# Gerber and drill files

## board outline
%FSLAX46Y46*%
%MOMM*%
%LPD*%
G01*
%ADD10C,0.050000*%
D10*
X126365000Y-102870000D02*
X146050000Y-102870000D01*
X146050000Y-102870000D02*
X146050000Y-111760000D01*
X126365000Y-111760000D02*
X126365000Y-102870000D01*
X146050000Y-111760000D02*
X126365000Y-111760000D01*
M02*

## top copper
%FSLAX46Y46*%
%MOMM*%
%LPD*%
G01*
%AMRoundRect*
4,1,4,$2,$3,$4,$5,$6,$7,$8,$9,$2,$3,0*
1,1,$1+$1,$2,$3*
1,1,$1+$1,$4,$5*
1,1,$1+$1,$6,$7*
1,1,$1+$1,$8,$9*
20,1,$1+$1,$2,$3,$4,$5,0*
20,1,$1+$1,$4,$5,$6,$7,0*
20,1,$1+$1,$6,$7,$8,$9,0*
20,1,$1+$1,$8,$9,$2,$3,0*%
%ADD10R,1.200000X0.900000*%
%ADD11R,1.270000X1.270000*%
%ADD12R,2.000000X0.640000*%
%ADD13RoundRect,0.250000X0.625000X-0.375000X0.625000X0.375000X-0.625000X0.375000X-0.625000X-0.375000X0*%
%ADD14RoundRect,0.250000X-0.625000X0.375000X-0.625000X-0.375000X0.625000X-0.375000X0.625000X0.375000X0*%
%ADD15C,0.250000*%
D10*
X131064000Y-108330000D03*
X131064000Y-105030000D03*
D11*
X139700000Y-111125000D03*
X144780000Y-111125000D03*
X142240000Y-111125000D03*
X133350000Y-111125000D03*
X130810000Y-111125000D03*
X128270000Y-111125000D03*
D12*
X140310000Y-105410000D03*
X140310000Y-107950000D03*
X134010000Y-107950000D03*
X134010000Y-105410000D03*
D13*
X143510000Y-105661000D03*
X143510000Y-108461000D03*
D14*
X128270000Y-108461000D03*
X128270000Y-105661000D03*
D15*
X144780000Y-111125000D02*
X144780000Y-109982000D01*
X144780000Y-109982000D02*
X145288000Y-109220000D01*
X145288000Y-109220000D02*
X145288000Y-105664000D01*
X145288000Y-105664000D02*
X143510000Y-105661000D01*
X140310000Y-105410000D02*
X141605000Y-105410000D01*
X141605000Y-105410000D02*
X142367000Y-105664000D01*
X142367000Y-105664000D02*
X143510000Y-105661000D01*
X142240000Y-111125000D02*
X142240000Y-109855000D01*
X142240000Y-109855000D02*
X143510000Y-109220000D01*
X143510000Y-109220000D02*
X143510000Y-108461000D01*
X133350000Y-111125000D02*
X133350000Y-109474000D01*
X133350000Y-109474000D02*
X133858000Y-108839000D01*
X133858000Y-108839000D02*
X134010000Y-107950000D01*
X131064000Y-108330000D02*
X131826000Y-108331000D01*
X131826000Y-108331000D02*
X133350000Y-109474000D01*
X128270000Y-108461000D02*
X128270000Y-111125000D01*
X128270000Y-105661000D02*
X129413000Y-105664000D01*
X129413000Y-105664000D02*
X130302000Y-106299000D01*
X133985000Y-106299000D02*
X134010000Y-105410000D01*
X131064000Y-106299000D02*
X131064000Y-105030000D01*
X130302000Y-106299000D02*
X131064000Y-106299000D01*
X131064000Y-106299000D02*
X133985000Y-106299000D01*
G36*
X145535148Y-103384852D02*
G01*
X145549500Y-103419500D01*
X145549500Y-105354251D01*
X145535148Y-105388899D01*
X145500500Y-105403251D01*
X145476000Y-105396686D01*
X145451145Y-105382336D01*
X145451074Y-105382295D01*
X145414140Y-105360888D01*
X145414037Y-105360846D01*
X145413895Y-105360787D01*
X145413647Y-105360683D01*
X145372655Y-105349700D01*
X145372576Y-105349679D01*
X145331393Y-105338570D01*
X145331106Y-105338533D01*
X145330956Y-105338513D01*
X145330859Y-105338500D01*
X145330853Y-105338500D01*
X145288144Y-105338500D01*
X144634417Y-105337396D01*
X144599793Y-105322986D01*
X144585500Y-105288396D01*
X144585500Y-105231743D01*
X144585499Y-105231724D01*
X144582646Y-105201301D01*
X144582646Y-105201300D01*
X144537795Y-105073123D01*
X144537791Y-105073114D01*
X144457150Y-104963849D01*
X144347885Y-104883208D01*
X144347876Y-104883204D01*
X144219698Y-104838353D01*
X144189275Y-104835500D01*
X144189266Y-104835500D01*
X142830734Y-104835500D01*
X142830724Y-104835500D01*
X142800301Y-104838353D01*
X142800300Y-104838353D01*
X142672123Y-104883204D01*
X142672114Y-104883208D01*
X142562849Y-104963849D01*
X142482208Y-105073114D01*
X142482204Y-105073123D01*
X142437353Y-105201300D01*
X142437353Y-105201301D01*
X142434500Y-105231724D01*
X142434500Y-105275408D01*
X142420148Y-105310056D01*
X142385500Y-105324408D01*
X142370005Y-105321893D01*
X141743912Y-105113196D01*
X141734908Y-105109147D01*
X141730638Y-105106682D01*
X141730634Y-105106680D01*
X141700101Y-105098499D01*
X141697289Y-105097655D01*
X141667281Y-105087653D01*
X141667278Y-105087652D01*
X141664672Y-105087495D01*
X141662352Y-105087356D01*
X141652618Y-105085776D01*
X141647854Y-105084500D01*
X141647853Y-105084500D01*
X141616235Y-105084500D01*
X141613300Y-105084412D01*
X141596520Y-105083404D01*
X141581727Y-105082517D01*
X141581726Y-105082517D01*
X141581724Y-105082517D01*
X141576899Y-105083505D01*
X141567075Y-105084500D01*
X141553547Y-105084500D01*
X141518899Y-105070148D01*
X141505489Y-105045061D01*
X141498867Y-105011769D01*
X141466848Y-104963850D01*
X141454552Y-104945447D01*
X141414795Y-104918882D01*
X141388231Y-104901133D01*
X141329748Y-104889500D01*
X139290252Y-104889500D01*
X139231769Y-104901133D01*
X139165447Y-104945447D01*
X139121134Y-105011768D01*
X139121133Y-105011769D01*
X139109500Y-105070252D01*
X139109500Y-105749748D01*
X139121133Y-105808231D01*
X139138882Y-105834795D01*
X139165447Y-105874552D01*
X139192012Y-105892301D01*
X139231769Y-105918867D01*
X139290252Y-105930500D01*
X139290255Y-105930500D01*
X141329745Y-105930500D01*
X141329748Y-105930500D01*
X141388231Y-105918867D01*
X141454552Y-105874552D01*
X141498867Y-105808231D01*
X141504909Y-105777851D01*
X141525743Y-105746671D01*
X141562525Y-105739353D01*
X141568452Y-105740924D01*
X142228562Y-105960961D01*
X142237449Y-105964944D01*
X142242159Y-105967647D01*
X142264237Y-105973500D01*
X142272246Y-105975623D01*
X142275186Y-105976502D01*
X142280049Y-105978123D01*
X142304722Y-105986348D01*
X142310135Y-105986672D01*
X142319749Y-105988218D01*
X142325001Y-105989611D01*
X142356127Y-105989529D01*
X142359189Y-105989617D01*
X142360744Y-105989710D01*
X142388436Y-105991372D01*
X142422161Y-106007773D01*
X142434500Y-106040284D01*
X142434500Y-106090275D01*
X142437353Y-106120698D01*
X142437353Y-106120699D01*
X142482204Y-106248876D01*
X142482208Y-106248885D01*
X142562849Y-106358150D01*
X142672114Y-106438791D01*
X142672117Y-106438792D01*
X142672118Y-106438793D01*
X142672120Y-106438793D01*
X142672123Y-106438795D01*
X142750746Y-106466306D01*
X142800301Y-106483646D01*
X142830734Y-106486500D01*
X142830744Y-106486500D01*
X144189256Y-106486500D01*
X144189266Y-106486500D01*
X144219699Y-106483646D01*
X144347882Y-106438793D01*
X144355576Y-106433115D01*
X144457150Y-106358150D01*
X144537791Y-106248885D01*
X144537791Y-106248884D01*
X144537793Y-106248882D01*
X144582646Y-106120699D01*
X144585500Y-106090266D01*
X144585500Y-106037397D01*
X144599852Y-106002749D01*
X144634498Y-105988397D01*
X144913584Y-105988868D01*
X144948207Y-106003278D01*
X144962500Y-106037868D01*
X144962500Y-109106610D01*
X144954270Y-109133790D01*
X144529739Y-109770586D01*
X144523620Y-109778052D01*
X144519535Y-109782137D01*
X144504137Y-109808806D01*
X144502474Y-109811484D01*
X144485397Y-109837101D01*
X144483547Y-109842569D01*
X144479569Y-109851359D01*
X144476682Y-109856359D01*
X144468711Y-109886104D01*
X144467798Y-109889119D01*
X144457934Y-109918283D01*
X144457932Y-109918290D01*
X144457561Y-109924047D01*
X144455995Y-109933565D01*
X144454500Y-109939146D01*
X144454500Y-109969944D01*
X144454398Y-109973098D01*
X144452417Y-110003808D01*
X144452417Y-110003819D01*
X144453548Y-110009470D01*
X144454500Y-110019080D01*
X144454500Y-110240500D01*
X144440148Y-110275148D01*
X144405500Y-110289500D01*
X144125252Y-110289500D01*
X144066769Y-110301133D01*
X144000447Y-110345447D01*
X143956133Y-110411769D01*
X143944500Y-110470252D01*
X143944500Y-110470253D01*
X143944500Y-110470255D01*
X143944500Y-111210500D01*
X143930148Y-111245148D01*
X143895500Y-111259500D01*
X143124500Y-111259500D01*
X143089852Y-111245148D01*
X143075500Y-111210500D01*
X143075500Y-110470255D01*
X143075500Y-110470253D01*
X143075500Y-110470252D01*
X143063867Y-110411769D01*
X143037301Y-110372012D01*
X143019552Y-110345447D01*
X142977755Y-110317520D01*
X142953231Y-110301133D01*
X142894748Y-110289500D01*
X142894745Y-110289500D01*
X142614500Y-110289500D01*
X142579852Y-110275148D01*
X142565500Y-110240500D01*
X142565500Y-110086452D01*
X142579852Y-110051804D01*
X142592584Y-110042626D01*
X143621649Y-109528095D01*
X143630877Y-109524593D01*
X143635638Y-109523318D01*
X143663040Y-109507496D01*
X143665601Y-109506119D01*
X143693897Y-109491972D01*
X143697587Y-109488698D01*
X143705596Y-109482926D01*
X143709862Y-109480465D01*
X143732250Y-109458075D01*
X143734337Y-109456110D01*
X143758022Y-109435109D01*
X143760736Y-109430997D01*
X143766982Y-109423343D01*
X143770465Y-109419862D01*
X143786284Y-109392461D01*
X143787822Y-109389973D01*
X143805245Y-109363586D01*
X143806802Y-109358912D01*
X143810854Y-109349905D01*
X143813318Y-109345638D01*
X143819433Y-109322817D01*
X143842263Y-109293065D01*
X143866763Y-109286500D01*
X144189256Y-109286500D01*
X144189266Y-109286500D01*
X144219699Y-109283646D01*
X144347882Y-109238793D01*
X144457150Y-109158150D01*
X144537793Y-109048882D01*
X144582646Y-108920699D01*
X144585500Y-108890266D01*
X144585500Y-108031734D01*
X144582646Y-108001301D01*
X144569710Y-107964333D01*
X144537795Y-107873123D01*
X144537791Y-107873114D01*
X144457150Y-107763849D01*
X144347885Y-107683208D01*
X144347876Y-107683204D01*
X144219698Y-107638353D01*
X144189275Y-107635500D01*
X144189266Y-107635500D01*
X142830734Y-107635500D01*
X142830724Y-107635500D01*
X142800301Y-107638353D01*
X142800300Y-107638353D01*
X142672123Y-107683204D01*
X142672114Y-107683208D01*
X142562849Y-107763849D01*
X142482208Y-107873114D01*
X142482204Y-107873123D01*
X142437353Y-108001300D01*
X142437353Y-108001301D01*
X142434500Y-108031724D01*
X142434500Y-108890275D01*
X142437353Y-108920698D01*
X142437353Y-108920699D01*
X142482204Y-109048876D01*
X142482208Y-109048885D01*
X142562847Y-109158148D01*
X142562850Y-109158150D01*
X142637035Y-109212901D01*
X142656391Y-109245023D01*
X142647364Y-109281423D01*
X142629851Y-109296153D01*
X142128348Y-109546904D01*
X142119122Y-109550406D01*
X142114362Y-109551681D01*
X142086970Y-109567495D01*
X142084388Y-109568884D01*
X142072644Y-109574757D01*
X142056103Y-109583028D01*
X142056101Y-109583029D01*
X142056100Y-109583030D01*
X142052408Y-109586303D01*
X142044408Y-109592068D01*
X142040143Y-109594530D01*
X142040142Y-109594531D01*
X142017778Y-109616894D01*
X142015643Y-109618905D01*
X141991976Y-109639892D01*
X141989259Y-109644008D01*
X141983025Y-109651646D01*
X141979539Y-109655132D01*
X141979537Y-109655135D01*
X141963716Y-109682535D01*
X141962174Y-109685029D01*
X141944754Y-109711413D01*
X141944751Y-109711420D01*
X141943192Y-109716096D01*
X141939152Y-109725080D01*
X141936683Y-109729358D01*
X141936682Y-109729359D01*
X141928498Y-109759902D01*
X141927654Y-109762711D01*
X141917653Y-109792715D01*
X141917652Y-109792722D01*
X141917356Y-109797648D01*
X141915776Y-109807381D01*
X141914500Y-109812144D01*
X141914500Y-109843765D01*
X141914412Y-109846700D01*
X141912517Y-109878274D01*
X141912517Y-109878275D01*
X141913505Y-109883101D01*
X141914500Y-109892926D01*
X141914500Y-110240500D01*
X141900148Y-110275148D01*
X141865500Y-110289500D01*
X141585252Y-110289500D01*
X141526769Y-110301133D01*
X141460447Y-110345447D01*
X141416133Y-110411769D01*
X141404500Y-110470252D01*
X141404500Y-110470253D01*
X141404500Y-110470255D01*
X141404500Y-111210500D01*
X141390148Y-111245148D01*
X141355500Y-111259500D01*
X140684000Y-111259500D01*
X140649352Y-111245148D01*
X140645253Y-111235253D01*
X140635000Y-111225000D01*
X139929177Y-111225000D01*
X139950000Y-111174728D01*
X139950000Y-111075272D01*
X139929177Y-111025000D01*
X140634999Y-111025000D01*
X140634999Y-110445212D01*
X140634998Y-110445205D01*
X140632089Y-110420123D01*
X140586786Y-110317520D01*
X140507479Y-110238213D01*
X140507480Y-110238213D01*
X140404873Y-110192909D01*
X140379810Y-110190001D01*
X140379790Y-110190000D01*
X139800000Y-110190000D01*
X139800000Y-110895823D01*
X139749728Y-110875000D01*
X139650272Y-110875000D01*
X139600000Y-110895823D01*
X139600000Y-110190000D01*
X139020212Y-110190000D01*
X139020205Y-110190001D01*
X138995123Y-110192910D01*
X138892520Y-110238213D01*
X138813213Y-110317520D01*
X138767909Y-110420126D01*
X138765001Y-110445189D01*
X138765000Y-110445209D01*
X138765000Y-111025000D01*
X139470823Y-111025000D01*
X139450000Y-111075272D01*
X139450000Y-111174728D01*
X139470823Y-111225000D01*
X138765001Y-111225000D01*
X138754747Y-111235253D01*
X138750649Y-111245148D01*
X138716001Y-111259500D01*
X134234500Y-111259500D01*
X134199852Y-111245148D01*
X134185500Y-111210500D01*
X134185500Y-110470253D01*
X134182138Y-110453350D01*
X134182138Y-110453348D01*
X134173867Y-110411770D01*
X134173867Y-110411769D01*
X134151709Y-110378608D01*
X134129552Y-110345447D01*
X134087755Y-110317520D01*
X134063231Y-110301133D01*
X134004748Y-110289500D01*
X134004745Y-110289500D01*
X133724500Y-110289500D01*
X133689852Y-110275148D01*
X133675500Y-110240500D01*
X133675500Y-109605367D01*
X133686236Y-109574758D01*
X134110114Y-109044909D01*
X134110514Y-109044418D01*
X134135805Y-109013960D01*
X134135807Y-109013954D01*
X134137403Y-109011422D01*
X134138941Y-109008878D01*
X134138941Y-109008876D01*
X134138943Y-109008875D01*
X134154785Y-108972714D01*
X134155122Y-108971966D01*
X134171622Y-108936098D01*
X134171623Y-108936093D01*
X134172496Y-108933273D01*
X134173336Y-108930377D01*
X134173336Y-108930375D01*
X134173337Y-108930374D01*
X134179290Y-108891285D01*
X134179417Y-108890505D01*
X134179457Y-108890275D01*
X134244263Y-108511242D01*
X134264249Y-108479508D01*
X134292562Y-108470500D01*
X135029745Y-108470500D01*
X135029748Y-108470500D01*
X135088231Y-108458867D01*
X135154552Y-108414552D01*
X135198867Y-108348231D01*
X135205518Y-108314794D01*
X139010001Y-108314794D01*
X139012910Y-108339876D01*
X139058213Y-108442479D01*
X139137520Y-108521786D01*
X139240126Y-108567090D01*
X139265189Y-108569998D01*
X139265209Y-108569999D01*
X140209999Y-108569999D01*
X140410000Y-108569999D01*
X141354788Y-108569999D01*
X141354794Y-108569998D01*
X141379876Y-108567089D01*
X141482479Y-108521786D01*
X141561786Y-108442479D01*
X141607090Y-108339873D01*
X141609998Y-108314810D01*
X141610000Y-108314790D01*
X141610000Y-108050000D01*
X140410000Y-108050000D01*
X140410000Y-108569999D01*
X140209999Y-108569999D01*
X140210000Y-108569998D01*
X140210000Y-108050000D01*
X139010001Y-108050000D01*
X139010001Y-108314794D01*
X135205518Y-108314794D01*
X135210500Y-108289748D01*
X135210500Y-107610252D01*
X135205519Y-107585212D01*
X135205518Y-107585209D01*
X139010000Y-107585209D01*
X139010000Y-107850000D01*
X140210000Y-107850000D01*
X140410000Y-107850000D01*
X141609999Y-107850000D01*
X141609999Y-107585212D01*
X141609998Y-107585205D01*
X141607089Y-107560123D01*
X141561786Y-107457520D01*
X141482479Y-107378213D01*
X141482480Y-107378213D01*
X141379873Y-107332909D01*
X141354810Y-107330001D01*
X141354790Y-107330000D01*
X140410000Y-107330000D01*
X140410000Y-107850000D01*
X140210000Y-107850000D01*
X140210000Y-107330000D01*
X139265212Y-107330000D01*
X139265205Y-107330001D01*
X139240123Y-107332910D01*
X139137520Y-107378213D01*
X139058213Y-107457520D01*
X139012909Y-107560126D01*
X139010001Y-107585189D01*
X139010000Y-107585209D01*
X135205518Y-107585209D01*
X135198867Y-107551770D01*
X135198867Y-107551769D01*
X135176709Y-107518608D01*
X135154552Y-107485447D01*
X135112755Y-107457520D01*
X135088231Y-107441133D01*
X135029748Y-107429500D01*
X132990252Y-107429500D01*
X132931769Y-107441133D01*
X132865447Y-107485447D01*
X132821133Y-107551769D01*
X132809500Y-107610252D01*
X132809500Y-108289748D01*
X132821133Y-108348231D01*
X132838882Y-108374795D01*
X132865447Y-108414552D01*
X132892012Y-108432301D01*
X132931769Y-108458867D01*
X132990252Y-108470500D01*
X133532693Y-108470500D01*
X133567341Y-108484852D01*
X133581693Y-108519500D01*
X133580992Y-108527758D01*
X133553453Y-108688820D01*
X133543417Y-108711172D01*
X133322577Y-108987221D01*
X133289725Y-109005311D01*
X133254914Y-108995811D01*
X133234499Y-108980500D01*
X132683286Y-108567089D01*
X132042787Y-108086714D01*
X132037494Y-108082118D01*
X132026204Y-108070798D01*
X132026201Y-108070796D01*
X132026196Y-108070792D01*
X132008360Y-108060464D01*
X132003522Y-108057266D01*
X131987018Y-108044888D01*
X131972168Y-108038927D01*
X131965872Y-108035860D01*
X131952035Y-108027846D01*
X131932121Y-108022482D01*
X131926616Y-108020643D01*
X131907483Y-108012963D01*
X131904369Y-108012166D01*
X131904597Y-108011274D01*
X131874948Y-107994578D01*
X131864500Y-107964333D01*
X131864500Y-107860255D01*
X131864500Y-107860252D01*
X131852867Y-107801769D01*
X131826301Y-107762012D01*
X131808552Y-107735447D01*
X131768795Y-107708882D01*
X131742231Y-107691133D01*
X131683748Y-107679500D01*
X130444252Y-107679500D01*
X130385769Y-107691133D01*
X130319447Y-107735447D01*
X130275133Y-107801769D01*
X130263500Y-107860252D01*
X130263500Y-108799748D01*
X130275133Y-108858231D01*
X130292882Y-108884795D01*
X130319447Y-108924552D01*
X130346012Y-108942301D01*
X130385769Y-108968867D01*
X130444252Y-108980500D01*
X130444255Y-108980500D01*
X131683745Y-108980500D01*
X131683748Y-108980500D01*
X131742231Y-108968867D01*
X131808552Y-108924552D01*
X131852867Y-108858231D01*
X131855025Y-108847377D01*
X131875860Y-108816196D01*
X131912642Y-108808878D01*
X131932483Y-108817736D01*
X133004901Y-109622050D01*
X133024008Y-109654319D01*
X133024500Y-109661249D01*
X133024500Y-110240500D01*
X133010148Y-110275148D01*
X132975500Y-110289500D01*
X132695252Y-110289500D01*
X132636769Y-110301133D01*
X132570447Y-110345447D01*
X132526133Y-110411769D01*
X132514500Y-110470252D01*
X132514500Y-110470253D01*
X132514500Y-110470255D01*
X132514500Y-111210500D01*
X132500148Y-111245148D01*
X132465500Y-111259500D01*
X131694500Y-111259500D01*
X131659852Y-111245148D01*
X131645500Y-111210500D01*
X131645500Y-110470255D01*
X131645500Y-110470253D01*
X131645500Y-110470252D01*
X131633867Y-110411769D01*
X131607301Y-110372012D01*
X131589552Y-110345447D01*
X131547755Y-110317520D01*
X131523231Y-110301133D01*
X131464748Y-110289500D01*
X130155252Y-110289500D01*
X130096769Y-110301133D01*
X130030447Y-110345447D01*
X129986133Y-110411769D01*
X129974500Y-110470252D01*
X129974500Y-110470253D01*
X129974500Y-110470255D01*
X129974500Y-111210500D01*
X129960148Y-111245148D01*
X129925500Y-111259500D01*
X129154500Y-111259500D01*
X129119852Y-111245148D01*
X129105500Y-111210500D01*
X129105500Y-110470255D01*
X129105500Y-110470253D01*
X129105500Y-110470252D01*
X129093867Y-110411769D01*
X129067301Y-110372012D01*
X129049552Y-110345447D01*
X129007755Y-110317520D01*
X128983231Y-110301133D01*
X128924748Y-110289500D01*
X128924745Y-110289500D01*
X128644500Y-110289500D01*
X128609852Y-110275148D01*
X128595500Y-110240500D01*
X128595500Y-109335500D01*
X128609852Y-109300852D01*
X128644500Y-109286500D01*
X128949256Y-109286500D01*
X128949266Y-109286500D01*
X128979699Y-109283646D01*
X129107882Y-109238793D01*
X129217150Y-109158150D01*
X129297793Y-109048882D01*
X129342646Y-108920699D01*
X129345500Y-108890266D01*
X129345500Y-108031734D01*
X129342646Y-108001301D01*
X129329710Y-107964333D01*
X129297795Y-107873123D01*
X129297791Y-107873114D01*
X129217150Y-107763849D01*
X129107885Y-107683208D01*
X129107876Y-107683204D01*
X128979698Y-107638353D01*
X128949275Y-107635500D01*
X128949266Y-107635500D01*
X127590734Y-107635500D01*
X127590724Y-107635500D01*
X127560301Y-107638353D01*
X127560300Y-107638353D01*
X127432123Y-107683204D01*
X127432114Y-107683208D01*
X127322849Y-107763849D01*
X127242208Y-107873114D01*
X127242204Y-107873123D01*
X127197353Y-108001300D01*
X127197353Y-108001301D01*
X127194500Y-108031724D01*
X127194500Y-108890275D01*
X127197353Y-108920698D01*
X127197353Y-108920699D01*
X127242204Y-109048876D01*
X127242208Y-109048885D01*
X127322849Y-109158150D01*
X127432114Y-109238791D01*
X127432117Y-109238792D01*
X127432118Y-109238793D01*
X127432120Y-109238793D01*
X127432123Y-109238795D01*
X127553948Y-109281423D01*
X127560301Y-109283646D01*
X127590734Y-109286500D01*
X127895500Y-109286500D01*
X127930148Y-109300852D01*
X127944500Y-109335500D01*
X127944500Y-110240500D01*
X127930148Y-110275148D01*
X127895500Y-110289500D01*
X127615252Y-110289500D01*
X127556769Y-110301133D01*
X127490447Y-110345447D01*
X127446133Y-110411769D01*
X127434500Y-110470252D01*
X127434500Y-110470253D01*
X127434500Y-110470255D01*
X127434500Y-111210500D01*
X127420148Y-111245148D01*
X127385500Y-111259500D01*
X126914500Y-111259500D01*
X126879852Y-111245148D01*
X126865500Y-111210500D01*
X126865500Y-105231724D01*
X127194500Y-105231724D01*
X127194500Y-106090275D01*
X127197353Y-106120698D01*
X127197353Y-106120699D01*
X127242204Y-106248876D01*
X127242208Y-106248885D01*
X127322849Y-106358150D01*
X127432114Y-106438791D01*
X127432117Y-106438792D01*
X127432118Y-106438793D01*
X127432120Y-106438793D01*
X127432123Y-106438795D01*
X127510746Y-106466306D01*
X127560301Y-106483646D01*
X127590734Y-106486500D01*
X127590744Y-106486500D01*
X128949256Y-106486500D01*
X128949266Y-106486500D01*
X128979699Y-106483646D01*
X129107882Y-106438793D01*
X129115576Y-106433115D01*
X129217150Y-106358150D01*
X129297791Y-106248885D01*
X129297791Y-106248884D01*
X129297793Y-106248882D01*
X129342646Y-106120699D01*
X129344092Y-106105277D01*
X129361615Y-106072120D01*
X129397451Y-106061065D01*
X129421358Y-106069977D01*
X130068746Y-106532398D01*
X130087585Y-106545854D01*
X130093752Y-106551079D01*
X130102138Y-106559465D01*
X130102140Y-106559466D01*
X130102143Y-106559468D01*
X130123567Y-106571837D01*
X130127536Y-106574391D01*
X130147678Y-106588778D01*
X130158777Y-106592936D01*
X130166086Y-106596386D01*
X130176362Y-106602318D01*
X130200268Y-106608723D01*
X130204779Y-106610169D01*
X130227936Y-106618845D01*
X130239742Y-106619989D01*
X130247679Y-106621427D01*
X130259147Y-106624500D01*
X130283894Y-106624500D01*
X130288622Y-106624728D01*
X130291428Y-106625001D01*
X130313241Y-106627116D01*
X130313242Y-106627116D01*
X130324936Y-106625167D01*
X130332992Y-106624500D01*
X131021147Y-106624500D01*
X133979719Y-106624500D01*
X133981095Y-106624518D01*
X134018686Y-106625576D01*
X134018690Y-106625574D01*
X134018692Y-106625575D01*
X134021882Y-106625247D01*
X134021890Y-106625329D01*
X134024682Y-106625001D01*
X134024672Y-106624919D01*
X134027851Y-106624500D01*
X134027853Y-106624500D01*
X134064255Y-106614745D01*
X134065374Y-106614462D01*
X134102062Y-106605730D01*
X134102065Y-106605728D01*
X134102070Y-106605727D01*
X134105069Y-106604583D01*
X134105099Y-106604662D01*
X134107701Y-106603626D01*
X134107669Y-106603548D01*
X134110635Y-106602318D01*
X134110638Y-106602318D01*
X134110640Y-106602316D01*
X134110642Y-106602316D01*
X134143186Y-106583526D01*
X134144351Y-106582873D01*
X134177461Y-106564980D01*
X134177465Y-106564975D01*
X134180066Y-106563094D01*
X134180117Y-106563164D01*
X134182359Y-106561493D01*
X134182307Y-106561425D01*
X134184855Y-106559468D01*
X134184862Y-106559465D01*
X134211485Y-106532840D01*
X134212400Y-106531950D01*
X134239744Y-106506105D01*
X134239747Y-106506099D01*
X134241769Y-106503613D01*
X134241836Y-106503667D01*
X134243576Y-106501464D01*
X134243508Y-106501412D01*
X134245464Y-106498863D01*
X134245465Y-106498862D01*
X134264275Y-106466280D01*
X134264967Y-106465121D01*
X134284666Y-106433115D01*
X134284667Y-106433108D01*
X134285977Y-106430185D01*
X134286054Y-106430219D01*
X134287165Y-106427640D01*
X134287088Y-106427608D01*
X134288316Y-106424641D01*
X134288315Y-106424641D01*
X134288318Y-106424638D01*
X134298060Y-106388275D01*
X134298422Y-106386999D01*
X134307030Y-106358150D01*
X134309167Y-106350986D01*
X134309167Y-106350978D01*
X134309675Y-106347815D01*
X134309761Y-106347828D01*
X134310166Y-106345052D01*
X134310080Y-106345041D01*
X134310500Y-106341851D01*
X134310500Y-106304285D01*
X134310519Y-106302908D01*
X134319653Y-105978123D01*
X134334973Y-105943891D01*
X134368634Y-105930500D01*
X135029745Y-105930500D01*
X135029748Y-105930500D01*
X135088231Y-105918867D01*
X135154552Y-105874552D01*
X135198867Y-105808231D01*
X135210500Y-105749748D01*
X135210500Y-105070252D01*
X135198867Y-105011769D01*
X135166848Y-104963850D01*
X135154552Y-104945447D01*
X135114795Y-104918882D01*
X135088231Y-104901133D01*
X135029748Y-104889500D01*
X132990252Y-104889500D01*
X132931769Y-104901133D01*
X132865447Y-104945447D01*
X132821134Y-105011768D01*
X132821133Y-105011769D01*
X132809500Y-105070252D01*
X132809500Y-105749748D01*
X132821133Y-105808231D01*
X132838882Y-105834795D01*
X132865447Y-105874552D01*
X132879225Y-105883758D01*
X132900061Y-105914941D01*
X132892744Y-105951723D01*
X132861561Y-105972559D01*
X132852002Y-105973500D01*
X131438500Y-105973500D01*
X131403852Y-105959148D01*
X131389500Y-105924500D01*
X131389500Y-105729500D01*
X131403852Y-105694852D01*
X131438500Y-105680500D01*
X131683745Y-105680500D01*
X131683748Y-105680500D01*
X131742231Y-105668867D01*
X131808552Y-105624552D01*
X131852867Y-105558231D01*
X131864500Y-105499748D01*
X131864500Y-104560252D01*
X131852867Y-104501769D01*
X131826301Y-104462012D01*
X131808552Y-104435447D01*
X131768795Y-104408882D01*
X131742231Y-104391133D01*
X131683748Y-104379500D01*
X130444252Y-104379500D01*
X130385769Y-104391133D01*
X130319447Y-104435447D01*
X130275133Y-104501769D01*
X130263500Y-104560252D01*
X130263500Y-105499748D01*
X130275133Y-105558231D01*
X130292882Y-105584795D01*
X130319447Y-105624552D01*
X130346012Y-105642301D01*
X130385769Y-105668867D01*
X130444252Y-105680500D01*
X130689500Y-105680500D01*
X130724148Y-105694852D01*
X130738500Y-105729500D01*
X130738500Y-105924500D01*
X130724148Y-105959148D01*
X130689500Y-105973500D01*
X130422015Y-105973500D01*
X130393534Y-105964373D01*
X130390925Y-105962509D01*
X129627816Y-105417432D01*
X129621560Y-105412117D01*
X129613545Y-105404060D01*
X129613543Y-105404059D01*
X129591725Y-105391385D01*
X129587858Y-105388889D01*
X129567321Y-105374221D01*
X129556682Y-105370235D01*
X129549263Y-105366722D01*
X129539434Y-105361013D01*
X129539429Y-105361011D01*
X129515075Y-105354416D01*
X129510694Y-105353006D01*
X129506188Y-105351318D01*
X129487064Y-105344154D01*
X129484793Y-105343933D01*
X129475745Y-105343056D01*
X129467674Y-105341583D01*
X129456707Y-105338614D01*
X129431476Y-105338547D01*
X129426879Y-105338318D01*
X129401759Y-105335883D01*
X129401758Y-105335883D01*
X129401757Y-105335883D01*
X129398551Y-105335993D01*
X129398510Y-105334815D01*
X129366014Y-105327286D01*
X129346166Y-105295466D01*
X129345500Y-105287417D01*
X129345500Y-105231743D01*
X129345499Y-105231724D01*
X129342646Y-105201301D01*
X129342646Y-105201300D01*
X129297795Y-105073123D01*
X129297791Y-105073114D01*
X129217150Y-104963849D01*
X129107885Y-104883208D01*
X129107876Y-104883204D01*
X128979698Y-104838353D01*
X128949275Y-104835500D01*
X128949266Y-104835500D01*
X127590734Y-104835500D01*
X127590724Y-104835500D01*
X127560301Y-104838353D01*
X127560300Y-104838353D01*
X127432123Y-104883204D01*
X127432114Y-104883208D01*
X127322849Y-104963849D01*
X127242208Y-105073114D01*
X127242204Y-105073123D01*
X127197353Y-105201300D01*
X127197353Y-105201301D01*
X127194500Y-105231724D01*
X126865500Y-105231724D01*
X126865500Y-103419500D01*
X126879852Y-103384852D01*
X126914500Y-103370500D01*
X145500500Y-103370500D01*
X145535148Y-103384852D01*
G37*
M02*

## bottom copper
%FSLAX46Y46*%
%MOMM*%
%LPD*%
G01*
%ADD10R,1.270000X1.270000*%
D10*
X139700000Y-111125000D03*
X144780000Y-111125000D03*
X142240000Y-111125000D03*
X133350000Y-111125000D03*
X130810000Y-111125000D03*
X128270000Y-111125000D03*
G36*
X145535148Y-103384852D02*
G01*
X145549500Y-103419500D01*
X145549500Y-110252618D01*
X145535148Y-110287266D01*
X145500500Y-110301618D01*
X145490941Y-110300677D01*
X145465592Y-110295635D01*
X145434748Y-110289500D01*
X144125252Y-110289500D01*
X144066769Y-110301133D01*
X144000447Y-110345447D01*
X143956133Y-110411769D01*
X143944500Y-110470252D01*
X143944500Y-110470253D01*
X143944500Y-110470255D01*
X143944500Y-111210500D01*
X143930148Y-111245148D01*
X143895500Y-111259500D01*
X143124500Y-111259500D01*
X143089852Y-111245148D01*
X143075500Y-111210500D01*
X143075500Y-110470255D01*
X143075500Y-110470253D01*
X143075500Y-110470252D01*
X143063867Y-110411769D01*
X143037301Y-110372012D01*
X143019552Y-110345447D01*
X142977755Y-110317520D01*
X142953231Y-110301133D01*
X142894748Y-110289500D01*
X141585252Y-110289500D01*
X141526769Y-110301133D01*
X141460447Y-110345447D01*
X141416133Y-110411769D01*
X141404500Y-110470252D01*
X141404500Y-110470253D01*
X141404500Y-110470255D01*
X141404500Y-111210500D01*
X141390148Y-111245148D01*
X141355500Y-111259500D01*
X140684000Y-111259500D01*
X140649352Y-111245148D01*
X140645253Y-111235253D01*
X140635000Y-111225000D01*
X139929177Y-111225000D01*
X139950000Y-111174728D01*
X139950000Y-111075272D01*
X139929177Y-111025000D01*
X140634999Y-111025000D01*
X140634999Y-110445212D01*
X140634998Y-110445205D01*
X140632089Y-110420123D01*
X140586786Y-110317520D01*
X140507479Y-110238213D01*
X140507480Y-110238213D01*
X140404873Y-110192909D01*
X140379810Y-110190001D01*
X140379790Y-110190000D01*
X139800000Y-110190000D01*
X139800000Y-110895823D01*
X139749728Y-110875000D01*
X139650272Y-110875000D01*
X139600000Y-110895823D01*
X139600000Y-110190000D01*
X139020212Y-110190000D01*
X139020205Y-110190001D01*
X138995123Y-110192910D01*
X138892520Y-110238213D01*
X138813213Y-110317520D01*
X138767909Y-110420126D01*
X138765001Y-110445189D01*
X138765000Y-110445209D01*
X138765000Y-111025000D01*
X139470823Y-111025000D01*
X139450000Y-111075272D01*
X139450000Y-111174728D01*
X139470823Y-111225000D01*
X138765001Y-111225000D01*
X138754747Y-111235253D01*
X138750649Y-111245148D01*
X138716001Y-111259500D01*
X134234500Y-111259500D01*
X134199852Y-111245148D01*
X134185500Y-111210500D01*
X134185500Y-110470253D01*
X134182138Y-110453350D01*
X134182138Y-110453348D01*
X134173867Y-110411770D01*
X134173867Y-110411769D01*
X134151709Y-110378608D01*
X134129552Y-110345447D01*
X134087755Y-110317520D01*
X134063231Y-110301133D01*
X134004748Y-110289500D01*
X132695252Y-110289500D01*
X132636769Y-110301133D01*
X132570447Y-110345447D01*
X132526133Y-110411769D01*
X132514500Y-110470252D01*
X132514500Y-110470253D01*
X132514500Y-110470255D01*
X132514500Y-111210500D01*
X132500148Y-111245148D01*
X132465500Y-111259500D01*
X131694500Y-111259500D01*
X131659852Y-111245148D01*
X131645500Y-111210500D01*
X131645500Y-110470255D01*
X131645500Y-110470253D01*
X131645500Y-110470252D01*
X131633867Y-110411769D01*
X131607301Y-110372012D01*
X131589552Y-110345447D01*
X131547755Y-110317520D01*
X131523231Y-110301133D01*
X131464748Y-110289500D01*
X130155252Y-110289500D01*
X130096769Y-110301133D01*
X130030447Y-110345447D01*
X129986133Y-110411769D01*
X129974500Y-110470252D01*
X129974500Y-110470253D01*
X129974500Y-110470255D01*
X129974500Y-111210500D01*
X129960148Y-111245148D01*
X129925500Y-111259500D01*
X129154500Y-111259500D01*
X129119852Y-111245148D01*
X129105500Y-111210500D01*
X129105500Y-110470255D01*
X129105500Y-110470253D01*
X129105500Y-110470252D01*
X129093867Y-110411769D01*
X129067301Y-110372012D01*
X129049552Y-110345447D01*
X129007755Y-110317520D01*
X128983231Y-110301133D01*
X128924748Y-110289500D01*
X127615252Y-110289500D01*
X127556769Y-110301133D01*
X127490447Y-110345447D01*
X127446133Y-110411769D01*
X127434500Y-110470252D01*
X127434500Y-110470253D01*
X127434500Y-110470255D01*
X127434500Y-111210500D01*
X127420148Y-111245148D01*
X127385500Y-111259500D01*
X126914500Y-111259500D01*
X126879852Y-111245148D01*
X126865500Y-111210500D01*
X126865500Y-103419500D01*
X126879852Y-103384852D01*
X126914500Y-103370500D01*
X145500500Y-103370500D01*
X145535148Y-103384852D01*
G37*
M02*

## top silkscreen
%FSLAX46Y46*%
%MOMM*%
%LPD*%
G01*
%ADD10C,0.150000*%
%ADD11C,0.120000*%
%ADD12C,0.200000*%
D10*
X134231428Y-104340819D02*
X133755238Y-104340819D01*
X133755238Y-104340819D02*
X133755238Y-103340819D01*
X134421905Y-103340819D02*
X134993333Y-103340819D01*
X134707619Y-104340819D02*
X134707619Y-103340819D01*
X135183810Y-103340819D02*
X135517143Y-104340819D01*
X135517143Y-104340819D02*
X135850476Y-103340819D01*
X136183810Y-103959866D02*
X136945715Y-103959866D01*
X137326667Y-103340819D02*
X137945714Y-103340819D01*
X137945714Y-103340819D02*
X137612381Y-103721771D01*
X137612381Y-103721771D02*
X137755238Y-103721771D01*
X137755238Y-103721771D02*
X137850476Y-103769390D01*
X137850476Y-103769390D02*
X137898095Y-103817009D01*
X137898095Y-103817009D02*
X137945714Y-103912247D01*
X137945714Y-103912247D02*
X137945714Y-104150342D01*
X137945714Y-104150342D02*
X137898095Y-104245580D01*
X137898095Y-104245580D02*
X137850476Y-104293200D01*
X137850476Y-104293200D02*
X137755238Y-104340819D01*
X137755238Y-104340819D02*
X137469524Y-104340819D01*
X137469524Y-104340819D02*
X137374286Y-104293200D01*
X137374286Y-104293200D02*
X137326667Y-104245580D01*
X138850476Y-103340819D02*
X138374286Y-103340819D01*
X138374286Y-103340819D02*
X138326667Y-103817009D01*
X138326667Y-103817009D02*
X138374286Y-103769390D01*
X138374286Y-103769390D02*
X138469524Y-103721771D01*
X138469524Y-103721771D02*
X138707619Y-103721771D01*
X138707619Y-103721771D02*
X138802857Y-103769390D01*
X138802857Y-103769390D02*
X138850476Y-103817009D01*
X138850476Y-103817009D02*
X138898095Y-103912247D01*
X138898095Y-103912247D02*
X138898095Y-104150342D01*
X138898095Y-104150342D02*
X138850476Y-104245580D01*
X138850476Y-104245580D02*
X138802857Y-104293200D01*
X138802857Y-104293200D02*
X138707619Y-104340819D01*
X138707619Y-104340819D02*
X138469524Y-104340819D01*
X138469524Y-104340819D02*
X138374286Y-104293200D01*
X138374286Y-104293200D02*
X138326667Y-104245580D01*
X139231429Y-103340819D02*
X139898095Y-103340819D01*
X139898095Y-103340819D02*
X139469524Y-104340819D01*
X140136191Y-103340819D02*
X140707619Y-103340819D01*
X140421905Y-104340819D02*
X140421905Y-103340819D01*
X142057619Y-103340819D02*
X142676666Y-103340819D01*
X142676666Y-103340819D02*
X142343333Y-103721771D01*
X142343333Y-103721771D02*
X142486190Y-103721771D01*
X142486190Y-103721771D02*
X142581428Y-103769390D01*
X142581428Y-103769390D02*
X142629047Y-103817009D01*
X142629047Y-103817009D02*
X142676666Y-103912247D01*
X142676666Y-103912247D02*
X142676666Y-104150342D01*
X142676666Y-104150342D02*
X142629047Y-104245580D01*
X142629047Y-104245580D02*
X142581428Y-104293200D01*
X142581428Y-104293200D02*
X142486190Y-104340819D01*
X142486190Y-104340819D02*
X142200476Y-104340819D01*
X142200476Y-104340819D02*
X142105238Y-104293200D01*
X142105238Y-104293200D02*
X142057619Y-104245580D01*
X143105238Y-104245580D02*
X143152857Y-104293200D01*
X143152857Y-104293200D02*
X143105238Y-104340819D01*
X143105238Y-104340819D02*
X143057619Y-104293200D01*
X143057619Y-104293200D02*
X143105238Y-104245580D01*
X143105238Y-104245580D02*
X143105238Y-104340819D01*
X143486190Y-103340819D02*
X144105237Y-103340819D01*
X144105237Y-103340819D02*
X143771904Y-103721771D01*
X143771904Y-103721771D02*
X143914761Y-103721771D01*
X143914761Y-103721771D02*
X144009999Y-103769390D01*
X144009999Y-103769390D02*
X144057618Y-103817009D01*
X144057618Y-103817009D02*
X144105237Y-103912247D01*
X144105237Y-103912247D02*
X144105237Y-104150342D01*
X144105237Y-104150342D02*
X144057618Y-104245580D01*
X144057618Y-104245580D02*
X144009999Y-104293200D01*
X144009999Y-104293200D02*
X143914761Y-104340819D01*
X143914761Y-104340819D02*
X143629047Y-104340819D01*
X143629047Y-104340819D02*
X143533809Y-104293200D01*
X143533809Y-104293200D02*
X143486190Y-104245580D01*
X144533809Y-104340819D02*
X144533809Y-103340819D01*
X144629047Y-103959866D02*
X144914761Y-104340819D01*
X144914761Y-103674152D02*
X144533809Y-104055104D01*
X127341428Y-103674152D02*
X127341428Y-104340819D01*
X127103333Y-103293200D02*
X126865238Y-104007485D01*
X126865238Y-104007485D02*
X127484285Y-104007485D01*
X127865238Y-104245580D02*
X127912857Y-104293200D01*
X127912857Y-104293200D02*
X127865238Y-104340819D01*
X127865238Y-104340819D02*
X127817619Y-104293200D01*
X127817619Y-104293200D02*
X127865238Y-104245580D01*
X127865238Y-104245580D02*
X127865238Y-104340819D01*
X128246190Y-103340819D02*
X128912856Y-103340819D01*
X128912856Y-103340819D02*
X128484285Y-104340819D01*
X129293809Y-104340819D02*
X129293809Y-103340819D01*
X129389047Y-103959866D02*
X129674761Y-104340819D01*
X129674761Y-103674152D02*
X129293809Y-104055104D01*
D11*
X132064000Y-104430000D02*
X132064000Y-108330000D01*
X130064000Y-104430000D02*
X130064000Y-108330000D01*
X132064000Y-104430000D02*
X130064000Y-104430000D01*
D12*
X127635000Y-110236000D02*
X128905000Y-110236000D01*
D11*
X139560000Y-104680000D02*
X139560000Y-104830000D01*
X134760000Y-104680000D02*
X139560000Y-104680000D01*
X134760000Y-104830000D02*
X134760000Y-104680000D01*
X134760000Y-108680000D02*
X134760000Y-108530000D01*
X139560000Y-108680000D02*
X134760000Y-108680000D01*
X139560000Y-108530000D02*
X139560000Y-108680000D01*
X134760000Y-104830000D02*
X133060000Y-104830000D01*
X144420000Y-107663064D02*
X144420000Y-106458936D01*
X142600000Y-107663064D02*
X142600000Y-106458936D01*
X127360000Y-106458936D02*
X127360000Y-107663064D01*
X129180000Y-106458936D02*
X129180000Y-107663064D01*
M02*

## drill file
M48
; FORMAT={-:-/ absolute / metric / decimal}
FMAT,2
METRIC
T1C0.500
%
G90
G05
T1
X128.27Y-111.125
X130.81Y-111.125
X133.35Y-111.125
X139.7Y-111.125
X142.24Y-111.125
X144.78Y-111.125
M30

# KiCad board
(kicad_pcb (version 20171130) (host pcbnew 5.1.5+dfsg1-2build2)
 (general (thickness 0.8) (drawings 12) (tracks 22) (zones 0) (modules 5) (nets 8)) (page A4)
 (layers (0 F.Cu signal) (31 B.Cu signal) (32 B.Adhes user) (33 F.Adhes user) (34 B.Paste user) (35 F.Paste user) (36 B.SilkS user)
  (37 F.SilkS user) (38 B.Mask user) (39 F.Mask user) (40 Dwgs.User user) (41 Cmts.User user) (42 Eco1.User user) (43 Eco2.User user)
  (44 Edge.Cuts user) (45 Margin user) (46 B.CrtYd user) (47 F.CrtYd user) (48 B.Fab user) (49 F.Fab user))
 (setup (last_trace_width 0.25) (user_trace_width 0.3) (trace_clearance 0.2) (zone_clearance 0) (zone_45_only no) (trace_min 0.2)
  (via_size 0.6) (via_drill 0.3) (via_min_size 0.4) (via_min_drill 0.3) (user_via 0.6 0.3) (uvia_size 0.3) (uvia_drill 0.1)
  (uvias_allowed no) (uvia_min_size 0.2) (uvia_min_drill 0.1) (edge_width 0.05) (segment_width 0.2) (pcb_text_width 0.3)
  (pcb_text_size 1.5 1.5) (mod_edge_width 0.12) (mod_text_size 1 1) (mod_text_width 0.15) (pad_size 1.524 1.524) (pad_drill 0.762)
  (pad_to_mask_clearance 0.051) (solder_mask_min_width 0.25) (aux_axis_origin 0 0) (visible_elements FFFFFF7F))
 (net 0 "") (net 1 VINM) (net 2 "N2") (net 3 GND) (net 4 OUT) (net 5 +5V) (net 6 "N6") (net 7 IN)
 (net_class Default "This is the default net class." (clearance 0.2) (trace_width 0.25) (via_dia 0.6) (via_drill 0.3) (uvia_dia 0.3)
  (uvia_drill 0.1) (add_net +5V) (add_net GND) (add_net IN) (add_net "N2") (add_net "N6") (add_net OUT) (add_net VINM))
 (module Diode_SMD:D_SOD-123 (layer F.Cu) (at 131.064 106.68 270)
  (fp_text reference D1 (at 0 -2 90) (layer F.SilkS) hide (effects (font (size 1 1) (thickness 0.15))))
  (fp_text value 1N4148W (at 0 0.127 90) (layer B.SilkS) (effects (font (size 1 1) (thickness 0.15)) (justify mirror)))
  (fp_line (start -2.25 -1) (end 1.65 -1) (layer F.SilkS) (width 0.12))
  (fp_line (start -2.25 1) (end 1.65 1) (layer F.SilkS) (width 0.12))
  (fp_line (start -2.25 -1) (end -2.25 1) (layer F.SilkS) (width 0.12))
  (pad 2 smd rect (at 1.65 0 270) (size 0.9 1.2) (layers F.Cu F.Paste F.Mask) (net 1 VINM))
  (pad 1 smd rect (at -1.65 0 270) (size 0.9 1.2) (layers F.Cu F.Paste F.Mask) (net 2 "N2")))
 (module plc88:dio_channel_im (layer F.Cu) (at 135.255 108.585)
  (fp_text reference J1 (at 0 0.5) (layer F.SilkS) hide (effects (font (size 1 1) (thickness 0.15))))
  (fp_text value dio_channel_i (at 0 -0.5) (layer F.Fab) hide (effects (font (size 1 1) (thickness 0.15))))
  (fp_line (start -7.62 1.651) (end -6.35 1.651) (layer F.SilkS) (width 0.2))
  (pad 4 thru_hole rect (at 4.445 2.54) (size 1.27 1.27) (drill 0.5) (layers *.Cu *.Mask) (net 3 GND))
  (pad 6 thru_hole rect (at 9.525 2.54) (size 1.27 1.27) (drill 0.5) (layers *.Cu *.Mask) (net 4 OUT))
  (pad 5 thru_hole rect (at 6.985 2.54) (size 1.27 1.27) (drill 0.5) (layers *.Cu *.Mask) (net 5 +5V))
  (pad 3 thru_hole rect (at -1.905 2.54) (size 1.27 1.27) (drill 0.5) (layers *.Cu *.Mask) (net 1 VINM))
  (pad 2 thru_hole rect (at -4.445 2.54) (size 1.27 1.27) (drill 0.5) (layers *.Cu *.Mask) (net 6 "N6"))
  (pad 1 thru_hole rect (at -6.985 2.54) (size 1.27 1.27) (drill 0.5) (layers *.Cu *.Mask) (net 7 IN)))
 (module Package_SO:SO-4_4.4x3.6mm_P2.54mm (layer F.Cu) (at 137.16 106.68)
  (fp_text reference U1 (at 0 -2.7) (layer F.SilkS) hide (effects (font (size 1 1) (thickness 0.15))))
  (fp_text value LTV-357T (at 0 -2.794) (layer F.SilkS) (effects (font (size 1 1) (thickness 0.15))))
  (fp_line (start 2.4 -2) (end 2.4 -1.85) (layer F.SilkS) (width 0.12))
  (fp_line (start -2.4 -2) (end 2.4 -2) (layer F.SilkS) (width 0.12))
  (fp_line (start -2.4 -1.85) (end -2.4 -2) (layer F.SilkS) (width 0.12))
  (fp_line (start -2.4 2) (end -2.4 1.85) (layer F.SilkS) (width 0.12))
  (fp_line (start 2.4 2) (end -2.4 2) (layer F.SilkS) (width 0.12))
  (fp_line (start 2.4 1.85) (end 2.4 2) (layer F.SilkS) (width 0.12))
  (fp_line (start -2.4 -1.85) (end -4.1 -1.85) (layer F.SilkS) (width 0.12))
  (pad 4 smd rect (at 3.15 -1.27) (size 2 0.64) (layers F.Cu F.Paste F.Mask) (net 4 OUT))
  (pad 3 smd rect (at 3.15 1.27) (size 2 0.64) (layers F.Cu F.Paste F.Mask) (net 3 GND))
  (pad 2 smd rect (at -3.15 1.27) (size 2 0.64) (layers F.Cu F.Paste F.Mask) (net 1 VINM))
  (pad 1 smd rect (at -3.15 -1.27) (size 2 0.64) (layers F.Cu F.Paste F.Mask) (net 2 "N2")))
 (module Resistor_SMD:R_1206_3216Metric (layer F.Cu) (at 143.51 107.061 90)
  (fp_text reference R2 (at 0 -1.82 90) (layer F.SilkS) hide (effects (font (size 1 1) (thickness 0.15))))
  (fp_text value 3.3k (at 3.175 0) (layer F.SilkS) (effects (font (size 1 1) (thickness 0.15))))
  (fp_line (start -0.602064 0.91) (end 0.602064 0.91) (layer F.SilkS) (width 0.12))
  (fp_line (start -0.602064 -0.91) (end 0.602064 -0.91) (layer F.SilkS) (width 0.12))
  (pad 2 smd roundrect (at 1.4 0 90) (size 1.25 1.75) (layers F.Cu F.Paste F.Mask) (roundrect_rratio 0.2) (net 4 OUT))
  (pad 1 smd roundrect (at -1.4 0 90) (size 1.25 1.75) (layers F.Cu F.Paste F.Mask) (roundrect_rratio 0.2) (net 5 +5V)))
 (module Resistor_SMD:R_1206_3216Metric (layer F.Cu) (at 128.27 107.061 270)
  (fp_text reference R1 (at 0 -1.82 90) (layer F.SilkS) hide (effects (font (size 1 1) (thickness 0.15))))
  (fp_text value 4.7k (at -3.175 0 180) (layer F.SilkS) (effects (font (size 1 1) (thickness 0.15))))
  (fp_line (start -0.602064 0.91) (end 0.602064 0.91) (layer F.SilkS) (width 0.12))
  (fp_line (start -0.602064 -0.91) (end 0.602064 -0.91) (layer F.SilkS) (width 0.12))
  (pad 2 smd roundrect (at 1.4 0 270) (size 1.25 1.75) (layers F.Cu F.Paste F.Mask) (roundrect_rratio 0.2) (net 7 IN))
  (pad 1 smd roundrect (at -1.4 0 270) (size 1.25 1.75) (layers F.Cu F.Paste F.Mask) (roundrect_rratio 0.2) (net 2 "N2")))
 (gr_line (start 126.365 102.87) (end 146.05 102.87) (layer Edge.Cuts) (width 0.05))
 (gr_line (start 146.05 102.87) (end 146.05 111.76) (layer Edge.Cuts) (width 0.05))
 (gr_line (start 126.365 111.76) (end 126.365 102.87) (layer Edge.Cuts) (width 0.05))
 (gr_line (start 146.05 111.76) (end 126.365 111.76) (layer Edge.Cuts) (width 0.05))
 (segment (start 144.78 111.125) (end 144.78 109.982) (width 0.25) (layer F.Cu) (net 4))
 (segment (start 144.78 109.982) (end 145.288 109.22) (width 0.25) (layer F.Cu) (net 4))
 (segment (start 145.288 109.22) (end 145.288 105.664) (width 0.25) (layer F.Cu) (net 4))
 (segment (start 145.288 105.664) (end 143.51 105.661) (width 0.25) (layer F.Cu) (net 4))
 (segment (start 140.31 105.41) (end 141.605 105.41) (width 0.25) (layer F.Cu) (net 4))
 (segment (start 141.605 105.41) (end 142.367 105.664) (width 0.25) (layer F.Cu) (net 4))
 (segment (start 142.367 105.664) (end 143.51 105.661) (width 0.25) (layer F.Cu) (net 4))
 (segment (start 142.24 111.125) (end 142.24 109.855) (width 0.25) (layer F.Cu) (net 5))
 (segment (start 142.24 109.855) (end 143.51 109.22) (width 0.25) (layer F.Cu) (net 5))
 (segment (start 143.51 109.22) (end 143.51 108.461) (width 0.25) (layer F.Cu) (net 5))
 (segment (start 133.35 111.125) (end 133.35 109.474) (width 0.25) (layer F.Cu) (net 1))
 (segment (start 133.35 109.474) (end 133.858 108.839) (width 0.25) (layer F.Cu) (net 1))
 (segment (start 133.858 108.839) (end 134.01 107.95) (width 0.25) (layer F.Cu) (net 1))
 (segment (start 131.064 108.33) (end 131.826 108.331) (width 0.25) (layer F.Cu) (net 1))
 (segment (start 131.826 108.331) (end 133.35 109.474) (width 0.25) (layer F.Cu) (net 1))
 (segment (start 128.27 108.461) (end 128.27 111.125) (width 0.25) (layer F.Cu) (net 7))
 (segment (start 128.27 105.661) (end 129.413 105.664) (width 0.25) (layer F.Cu) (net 2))
 (segment (start 129.413 105.664) (end 130.302 106.299) (width 0.25) (layer F.Cu) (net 2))
 (segment (start 133.985 106.299) (end 134.01 105.41) (width 0.25) (layer F.Cu) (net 2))
 (segment (start 131.064 106.299) (end 131.064 105.03) (width 0.25) (layer F.Cu) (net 2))
 (segment (start 130.302 106.299) (end 131.064 106.299) (width 0.25) (layer F.Cu) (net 2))
 (segment (start 131.064 106.299) (end 133.985 106.299) (width 0.25) (layer F.Cu) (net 2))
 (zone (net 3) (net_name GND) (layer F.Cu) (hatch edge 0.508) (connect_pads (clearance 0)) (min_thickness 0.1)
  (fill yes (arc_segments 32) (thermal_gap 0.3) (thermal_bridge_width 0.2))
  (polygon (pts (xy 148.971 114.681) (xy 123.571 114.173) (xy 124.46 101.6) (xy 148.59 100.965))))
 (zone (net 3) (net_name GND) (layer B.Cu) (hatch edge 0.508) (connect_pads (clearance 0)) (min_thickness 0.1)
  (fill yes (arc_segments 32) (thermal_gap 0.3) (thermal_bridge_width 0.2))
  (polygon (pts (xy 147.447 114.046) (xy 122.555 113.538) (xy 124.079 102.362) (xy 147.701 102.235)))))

